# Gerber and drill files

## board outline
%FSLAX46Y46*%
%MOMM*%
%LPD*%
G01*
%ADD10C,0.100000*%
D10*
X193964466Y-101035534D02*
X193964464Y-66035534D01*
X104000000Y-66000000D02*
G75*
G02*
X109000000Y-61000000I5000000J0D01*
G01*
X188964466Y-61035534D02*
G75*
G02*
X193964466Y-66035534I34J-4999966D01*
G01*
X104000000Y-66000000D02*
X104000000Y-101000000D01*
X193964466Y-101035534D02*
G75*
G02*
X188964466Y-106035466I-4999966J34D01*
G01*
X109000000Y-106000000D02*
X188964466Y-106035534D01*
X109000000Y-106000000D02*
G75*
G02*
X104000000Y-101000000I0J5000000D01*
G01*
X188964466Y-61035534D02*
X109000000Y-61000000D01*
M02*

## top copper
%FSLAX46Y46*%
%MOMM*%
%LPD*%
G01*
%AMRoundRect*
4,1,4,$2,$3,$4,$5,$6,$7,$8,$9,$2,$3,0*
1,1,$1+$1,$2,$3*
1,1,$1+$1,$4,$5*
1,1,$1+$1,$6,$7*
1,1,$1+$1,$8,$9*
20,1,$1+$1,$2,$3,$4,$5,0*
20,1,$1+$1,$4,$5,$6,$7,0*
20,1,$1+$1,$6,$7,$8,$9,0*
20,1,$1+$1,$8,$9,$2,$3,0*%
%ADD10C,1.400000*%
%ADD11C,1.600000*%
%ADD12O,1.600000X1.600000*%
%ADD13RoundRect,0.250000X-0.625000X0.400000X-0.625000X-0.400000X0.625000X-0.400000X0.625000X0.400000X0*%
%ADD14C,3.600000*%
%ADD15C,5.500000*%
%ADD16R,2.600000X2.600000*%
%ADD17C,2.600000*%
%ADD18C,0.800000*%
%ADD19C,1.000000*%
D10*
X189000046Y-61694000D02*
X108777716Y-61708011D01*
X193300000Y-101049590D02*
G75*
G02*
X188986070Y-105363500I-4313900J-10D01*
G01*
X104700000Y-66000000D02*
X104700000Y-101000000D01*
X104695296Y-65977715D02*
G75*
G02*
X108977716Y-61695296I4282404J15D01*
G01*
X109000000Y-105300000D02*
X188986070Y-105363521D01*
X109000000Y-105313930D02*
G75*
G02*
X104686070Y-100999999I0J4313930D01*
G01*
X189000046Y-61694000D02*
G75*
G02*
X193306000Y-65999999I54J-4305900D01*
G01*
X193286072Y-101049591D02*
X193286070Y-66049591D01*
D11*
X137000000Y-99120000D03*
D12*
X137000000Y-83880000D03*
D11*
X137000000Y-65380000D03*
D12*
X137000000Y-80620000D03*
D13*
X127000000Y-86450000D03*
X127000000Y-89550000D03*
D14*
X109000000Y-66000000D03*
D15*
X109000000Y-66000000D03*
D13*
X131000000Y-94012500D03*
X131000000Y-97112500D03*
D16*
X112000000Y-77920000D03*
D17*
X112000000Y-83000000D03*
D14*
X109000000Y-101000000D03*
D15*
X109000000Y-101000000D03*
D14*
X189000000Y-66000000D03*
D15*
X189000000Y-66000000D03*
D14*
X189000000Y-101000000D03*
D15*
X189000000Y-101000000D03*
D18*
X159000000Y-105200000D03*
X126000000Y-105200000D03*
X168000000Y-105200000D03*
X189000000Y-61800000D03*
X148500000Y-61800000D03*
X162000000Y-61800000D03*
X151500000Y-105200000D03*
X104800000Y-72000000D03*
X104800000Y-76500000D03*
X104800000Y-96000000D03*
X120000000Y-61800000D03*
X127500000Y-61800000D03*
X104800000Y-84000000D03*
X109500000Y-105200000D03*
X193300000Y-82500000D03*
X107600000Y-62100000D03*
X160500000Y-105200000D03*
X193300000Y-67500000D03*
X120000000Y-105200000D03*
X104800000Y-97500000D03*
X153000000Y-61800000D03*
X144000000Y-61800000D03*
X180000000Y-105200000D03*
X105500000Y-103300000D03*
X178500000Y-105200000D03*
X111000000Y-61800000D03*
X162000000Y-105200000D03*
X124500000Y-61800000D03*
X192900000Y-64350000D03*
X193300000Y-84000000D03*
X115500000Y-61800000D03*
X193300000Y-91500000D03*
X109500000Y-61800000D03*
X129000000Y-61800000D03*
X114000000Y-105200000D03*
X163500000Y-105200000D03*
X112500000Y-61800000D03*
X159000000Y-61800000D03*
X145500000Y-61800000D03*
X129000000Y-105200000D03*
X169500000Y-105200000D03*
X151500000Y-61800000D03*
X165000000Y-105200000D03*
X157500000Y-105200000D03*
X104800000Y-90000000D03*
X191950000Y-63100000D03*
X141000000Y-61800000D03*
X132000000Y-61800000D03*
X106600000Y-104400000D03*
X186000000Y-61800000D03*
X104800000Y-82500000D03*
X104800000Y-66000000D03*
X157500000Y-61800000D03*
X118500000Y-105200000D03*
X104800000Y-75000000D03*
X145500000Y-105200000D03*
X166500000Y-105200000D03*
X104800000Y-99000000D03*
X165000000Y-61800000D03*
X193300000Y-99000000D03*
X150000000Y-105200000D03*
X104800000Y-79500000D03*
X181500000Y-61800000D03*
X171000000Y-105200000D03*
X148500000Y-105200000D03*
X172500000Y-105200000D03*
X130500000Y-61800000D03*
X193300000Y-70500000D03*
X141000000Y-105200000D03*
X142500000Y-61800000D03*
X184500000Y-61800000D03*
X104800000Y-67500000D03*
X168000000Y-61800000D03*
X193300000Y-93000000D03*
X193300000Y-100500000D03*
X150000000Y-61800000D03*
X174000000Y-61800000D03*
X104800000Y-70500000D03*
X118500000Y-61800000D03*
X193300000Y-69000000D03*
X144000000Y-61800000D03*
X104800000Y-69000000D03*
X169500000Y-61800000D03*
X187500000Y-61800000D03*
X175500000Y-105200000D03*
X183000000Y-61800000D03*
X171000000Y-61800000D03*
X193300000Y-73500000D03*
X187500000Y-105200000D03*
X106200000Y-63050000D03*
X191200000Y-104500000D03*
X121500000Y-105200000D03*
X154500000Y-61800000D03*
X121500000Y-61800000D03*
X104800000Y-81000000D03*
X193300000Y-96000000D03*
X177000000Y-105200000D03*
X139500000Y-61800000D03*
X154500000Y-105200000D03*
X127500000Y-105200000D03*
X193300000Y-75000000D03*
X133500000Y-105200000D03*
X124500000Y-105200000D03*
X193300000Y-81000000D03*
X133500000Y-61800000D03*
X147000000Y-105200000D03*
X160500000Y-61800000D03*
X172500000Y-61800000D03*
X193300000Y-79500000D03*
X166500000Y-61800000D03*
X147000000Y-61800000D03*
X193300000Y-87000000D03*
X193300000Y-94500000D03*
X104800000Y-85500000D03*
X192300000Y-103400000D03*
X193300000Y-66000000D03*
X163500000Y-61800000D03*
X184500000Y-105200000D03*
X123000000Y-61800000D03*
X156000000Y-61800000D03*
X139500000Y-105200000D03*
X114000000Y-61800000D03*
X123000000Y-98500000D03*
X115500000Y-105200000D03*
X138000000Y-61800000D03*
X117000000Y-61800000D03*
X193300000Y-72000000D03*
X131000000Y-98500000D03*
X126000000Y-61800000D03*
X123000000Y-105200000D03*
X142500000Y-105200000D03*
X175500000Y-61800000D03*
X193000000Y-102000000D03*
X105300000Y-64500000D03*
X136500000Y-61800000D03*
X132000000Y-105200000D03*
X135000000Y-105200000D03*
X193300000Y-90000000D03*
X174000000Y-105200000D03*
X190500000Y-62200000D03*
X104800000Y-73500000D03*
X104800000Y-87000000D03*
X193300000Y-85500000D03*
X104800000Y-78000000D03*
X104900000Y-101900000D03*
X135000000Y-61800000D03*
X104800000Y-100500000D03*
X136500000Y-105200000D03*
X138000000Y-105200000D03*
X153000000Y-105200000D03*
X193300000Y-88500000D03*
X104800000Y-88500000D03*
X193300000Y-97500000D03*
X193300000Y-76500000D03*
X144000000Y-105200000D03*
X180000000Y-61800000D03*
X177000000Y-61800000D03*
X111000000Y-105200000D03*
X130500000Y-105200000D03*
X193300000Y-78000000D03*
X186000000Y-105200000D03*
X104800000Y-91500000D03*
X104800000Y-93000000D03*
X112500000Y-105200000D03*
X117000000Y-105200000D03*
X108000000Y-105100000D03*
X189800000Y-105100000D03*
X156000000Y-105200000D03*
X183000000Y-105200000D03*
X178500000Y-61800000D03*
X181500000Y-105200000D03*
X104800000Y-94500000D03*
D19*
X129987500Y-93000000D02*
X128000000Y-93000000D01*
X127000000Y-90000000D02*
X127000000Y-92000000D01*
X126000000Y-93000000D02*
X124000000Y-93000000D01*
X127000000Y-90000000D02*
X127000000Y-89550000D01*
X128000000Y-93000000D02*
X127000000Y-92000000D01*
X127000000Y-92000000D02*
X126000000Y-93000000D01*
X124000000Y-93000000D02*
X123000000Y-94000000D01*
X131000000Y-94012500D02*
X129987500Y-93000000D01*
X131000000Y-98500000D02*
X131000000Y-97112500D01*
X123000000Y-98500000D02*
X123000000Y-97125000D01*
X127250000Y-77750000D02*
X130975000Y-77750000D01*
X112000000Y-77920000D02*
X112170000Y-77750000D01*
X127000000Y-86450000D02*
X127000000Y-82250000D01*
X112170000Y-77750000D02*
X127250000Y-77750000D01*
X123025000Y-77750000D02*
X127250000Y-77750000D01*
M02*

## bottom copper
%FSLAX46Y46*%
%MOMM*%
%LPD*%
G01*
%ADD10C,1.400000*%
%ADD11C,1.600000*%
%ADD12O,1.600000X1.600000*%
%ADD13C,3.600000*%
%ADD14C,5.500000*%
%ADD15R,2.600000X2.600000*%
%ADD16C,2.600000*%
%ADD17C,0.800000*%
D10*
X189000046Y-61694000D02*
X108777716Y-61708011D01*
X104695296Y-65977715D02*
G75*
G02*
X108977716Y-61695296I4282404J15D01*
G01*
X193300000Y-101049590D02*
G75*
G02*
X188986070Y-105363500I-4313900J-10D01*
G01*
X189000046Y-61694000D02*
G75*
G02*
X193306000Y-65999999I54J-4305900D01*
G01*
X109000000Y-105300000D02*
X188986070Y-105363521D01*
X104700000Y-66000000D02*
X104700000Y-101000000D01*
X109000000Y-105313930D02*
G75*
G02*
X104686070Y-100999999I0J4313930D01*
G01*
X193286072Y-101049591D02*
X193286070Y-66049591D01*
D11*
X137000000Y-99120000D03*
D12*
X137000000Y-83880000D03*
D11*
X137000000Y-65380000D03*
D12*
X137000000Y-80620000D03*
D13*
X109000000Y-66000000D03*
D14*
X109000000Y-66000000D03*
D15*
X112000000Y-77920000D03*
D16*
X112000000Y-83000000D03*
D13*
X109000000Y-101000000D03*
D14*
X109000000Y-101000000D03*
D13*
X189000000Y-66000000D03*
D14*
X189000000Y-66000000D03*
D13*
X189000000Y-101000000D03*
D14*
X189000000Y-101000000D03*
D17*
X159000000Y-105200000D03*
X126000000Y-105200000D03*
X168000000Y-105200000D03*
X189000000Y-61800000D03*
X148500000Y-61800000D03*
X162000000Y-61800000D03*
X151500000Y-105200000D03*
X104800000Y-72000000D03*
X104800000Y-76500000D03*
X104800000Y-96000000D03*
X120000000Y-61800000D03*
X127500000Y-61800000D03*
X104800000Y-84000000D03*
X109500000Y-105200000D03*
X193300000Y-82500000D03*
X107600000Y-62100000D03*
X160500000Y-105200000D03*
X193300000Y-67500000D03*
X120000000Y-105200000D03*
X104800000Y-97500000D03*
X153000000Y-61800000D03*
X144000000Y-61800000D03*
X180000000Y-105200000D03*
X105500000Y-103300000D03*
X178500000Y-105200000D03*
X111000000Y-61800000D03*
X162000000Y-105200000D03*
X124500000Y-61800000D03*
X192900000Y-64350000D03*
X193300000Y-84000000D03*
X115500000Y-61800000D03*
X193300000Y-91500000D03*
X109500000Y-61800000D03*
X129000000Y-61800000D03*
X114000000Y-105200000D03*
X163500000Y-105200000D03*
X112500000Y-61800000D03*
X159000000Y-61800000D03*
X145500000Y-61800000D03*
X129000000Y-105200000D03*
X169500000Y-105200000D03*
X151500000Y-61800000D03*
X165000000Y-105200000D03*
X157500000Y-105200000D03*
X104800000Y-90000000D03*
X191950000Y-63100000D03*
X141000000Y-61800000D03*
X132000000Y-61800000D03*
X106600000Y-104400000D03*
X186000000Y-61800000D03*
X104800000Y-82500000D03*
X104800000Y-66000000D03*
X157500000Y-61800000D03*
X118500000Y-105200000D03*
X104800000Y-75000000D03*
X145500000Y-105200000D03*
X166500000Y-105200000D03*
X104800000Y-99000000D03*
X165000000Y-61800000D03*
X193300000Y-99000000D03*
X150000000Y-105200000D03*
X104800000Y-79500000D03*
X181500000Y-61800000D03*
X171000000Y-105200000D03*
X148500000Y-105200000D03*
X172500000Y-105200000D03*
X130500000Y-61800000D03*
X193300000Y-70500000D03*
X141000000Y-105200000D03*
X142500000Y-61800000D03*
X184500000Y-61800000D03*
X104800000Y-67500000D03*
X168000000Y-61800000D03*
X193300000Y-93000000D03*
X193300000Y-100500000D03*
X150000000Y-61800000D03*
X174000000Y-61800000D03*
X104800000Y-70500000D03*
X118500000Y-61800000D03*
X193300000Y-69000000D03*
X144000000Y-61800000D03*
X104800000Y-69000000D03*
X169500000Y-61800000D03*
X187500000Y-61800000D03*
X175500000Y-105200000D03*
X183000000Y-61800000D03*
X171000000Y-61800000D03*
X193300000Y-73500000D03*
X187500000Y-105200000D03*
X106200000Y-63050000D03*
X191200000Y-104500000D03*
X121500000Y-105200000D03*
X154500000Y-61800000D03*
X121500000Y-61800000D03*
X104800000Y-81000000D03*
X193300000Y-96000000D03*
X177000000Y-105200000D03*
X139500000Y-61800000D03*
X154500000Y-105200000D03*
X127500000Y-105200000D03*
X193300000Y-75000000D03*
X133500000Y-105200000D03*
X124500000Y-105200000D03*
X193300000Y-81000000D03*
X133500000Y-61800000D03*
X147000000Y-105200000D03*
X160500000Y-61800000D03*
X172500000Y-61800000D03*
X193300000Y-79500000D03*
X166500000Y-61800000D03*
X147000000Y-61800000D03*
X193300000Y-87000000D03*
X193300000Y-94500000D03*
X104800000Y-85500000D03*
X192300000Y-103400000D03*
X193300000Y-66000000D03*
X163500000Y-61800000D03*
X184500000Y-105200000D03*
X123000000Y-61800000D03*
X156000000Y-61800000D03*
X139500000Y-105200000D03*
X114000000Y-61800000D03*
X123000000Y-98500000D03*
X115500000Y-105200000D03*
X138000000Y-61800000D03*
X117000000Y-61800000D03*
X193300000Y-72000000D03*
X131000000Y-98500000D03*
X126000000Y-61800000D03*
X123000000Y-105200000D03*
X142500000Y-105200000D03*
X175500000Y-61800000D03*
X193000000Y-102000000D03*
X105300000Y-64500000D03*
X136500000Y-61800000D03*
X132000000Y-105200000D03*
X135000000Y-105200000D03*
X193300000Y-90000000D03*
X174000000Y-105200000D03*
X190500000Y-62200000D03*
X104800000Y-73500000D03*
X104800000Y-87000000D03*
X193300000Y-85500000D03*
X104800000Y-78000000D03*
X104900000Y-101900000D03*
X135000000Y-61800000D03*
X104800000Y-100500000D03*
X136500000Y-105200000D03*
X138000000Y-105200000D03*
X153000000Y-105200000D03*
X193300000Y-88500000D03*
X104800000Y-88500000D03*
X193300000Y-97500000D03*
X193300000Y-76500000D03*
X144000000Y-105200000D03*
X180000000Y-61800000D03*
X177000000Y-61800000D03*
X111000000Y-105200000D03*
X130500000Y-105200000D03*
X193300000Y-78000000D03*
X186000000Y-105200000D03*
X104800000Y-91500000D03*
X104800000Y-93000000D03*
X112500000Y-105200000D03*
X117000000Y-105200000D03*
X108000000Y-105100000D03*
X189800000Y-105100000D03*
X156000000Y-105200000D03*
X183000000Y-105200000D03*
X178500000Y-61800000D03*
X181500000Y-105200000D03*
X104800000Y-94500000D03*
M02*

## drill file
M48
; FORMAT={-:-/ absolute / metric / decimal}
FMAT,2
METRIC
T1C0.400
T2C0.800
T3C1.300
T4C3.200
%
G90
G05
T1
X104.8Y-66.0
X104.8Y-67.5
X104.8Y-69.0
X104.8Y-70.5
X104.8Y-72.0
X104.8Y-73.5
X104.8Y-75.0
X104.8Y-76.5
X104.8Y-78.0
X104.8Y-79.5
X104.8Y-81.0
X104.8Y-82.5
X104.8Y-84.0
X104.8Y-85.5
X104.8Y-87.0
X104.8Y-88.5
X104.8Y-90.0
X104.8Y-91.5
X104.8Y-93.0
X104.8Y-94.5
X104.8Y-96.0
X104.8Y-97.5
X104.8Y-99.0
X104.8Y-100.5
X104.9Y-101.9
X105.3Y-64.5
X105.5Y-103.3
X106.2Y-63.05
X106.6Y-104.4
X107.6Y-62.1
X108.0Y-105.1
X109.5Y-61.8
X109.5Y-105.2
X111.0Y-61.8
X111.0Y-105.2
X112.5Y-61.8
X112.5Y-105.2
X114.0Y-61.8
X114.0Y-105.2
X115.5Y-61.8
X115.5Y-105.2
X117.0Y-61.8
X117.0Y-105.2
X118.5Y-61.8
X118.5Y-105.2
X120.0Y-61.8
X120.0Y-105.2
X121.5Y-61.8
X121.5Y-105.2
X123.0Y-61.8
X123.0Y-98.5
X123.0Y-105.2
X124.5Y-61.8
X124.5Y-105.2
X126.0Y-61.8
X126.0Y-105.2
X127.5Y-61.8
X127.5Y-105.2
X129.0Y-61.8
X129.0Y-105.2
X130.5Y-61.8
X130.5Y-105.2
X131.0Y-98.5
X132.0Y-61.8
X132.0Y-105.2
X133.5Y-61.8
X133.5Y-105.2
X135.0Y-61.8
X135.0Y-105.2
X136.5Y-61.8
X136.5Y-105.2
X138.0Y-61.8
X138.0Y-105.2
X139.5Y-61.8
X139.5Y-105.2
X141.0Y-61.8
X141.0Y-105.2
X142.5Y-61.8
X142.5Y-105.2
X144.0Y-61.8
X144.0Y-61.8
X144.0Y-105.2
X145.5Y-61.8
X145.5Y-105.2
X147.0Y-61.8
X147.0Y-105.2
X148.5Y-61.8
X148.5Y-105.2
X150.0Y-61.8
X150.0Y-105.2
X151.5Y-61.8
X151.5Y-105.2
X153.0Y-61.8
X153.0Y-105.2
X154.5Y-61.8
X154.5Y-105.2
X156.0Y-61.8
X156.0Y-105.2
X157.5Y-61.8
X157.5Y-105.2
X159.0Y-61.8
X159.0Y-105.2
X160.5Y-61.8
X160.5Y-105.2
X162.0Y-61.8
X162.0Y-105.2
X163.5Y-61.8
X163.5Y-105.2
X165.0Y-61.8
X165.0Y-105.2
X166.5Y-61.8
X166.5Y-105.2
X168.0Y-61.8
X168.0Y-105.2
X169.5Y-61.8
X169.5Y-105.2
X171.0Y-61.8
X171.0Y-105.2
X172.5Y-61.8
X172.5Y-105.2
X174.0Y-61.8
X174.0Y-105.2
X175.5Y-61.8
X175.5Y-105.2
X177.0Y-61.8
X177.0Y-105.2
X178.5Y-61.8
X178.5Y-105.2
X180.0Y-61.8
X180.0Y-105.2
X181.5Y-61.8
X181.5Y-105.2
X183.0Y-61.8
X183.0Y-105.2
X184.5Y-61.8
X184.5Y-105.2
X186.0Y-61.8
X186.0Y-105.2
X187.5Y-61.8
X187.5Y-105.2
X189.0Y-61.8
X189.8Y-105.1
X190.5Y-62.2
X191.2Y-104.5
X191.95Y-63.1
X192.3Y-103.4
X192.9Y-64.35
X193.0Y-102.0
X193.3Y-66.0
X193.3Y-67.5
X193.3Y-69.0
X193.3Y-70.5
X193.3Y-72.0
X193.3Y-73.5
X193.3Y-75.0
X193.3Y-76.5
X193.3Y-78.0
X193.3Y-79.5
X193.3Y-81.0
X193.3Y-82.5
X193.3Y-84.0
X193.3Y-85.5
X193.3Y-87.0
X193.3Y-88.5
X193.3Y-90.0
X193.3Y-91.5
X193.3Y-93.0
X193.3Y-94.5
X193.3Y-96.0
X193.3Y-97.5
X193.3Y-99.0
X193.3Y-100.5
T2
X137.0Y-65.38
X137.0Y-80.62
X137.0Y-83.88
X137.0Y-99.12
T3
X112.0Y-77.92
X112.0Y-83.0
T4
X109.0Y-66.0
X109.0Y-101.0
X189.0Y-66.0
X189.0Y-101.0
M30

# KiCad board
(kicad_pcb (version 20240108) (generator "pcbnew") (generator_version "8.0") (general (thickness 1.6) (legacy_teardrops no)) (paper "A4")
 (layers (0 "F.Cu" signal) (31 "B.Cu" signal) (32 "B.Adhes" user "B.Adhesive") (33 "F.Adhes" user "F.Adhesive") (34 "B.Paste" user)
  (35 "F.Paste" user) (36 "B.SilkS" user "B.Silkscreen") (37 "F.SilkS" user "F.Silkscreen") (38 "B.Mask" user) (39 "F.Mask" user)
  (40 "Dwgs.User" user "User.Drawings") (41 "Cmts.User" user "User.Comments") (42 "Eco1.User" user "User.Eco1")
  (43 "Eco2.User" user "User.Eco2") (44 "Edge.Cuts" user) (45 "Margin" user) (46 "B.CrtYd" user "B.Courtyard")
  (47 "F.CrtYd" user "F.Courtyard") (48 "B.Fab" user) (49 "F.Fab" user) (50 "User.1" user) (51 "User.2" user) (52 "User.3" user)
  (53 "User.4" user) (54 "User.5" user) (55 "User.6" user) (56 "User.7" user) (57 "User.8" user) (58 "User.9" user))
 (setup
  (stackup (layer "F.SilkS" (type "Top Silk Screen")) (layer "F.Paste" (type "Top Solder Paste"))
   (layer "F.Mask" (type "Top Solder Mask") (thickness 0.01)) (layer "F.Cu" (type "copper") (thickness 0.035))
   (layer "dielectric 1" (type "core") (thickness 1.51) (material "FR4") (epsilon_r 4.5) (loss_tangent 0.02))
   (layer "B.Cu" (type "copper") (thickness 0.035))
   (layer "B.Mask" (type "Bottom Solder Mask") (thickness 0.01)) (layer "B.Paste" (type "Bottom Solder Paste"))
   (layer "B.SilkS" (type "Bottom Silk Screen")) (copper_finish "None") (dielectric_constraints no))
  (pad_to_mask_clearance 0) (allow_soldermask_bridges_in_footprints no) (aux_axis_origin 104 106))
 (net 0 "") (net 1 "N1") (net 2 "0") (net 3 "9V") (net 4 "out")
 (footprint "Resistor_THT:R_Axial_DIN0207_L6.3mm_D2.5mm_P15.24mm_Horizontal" (layer "F.Cu") (at 137 99.12 90)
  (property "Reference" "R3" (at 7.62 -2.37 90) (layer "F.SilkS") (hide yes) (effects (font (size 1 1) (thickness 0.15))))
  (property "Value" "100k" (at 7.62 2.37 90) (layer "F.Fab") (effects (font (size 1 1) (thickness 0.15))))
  (pad "1" thru_hole circle (at 0 0 90) (size 1.6 1.6) (drill 0.8) (layers "*.Cu" "*.Mask") (remove_unused_layers no) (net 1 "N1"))
  (pad "2" thru_hole oval (at 15.24 0 90) (size 1.6 1.6) (drill 0.8) (layers "*.Cu" "*.Mask") (remove_unused_layers no) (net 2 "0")))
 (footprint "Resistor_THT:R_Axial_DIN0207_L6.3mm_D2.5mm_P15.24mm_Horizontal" (layer "F.Cu") (at 137 65.38 -90)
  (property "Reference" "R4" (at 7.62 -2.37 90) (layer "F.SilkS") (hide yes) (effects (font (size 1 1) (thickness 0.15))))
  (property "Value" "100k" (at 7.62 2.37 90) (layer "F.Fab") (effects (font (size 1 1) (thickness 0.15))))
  (pad "1" thru_hole circle (at 0 0 270) (size 1.6 1.6) (drill 0.8) (layers "*.Cu" "*.Mask") (remove_unused_layers no) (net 1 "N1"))
  (pad "2" thru_hole oval (at 15.24 0 270) (size 1.6 1.6) (drill 0.8) (layers "*.Cu" "*.Mask") (remove_unused_layers no) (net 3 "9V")))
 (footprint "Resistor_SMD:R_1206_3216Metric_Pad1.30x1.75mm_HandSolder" (layer "F.Cu") (at 127 88 -90)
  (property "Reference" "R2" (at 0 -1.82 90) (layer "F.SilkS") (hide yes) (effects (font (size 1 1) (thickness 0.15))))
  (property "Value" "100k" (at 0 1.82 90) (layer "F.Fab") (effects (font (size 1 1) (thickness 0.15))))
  (pad "1" smd roundrect (at -1.55 0 270) (size 1.3 1.75) (layers "F.Cu" "F.Paste" "F.Mask") (roundrect_rratio 0.1923076923) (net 3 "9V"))
  (pad "2" smd roundrect (at 1.55 0 270) (size 1.3 1.75) (layers "F.Cu" "F.Paste" "F.Mask") (roundrect_rratio 0.1923076923) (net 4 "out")))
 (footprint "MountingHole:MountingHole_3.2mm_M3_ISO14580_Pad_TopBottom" (layer "F.Cu") (at 109 66)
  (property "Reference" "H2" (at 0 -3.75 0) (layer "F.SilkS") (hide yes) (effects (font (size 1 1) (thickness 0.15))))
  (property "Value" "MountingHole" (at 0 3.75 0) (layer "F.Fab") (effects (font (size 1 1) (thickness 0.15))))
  (pad "1" thru_hole circle (at 0 0) (size 3.6 3.6) (drill 3.2) (layers "*.Cu" "*.Mask") (remove_unused_layers no))
  (pad "1" connect circle (at 0 0) (size 5.5 5.5) (layers "F.Cu" "F.Mask"))
  (pad "1" connect circle (at 0 0) (size 5.5 5.5) (layers "B.Cu" "B.Mask")))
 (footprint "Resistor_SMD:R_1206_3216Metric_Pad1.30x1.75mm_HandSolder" (layer "F.Cu") (at 131 95.5625 -90)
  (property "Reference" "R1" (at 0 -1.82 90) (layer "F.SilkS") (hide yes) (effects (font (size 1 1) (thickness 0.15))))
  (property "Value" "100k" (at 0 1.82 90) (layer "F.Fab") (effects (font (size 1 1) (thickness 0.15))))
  (pad "1" smd roundrect (at -1.55 0 270) (size 1.3 1.75) (layers "F.Cu" "F.Paste" "F.Mask") (roundrect_rratio 0.1923076923) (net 4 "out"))
  (pad "2" smd roundrect (at 1.55 0 270) (size 1.3 1.75) (layers "F.Cu" "F.Paste" "F.Mask") (roundrect_rratio 0.1923076923) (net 2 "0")))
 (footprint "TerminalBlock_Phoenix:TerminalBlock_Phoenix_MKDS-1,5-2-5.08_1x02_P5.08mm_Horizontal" (layer "F.Cu") (at 112 77.92 -90)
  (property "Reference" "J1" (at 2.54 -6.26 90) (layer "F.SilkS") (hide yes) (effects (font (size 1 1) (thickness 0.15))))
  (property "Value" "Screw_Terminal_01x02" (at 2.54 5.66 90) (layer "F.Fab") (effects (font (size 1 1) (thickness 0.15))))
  (pad "1" thru_hole rect (at 0 0 270) (size 2.6 2.6) (drill 1.3) (layers "*.Cu" "*.Mask") (remove_unused_layers no) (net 3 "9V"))
  (pad "2" thru_hole circle (at 5.08 0 270) (size 2.6 2.6) (drill 1.3) (layers "*.Cu" "*.Mask") (remove_unused_layers no) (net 2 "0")))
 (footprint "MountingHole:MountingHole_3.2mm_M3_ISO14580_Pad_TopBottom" (layer "F.Cu") (at 109 101 -90)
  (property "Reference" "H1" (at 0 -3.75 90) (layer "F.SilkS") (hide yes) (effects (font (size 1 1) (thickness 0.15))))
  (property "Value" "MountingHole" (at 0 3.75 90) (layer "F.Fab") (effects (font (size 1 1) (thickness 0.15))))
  (pad "1" thru_hole circle (at 0 0 270) (size 3.6 3.6) (drill 3.2) (layers "*.Cu" "*.Mask") (remove_unused_layers no))
  (pad "1" connect circle (at 0 0 270) (size 5.5 5.5) (layers "F.Cu" "F.Mask"))
  (pad "1" connect circle (at 0 0 270) (size 5.5 5.5) (layers "B.Cu" "B.Mask")))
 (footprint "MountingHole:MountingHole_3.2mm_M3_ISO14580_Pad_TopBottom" (layer "F.Cu") (at 189 66)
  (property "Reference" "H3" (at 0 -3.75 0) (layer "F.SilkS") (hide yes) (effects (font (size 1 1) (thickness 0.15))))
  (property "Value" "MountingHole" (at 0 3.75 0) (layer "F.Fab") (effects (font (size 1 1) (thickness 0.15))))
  (pad "1" thru_hole circle (at 0 0) (size 3.6 3.6) (drill 3.2) (layers "*.Cu" "*.Mask") (remove_unused_layers no))
  (pad "1" connect circle (at 0 0) (size 5.5 5.5) (layers "F.Cu" "F.Mask"))
  (pad "1" connect circle (at 0 0) (size 5.5 5.5) (layers "B.Cu" "B.Mask")))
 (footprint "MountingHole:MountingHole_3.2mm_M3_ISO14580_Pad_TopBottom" (layer "F.Cu") (at 189 101)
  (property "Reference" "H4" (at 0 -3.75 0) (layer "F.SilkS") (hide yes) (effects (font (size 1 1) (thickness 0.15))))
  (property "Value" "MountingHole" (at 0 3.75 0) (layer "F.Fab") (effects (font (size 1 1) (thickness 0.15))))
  (pad "1" thru_hole circle (at 0 0) (size 3.6 3.6) (drill 3.2) (layers "*.Cu" "*.Mask") (remove_unused_layers no))
  (pad "1" connect circle (at 0 0) (size 5.5 5.5) (layers "F.Cu" "F.Mask"))
  (pad "1" connect circle (at 0 0) (size 5.5 5.5) (layers "B.Cu" "B.Mask")))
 (gr_line (start 189.000046 61.694) (end 108.777716 61.708011) (stroke (width 1.4) (type default)) (layer "F.Cu") (net 2))
 (gr_arc (start 193.3 101.04959) (mid 192.036477 104.099991) (end 188.98607 105.363521) (stroke (width 1.4) (type default)) (layer "F.Cu")
  (net 2))
 (gr_line (start 104.7 66) (end 104.7 101) (stroke (width 1.4) (type default)) (layer "F.Cu") (net 2))
 (gr_arc (start 104.695296 65.977715) (mid 105.949583 62.949583) (end 108.977716 61.695296) (stroke (width 1.4) (type default))
  (layer "F.Cu") (net 2))
 (gr_line (start 109 105.3) (end 188.98607 105.363521) (stroke (width 1.4) (type default)) (layer "F.Cu") (net 2))
 (gr_arc (start 109 105.31393) (mid 105.949588 104.05041) (end 104.68607 100.999999) (stroke (width 1.4) (type default)) (layer "F.Cu")
  (net 2))
 (gr_arc (start 189.000046 61.694) (mid 192.04487 62.955184) (end 193.306046 65.999999) (stroke (width 1.4) (type default)) (layer "F.Cu")
  (net 2))
 (gr_line (start 193.286072 101.049591) (end 193.28607 66.049591) (stroke (width 1.4) (type default)) (layer "F.Cu") (net 2))
 (gr_line (start 189.000046 61.694) (end 108.777716 61.708011) (stroke (width 1.4) (type default)) (layer "B.Cu") (net 2))
 (gr_arc (start 104.695296 65.977715) (mid 105.949583 62.949583) (end 108.977716 61.695296) (stroke (width 1.4) (type default))
  (layer "B.Cu") (net 2))
 (gr_arc (start 193.3 101.04959) (mid 192.036477 104.099991) (end 188.98607 105.363521) (stroke (width 1.4) (type default)) (layer "B.Cu")
  (net 2))
 (gr_arc (start 189.000046 61.694) (mid 192.04487 62.955184) (end 193.306046 65.999999) (stroke (width 1.4) (type default)) (layer "B.Cu")
  (net 2))
 (gr_line (start 109 105.3) (end 188.98607 105.363521) (stroke (width 1.4) (type default)) (layer "B.Cu") (net 2))
 (gr_line (start 104.7 66) (end 104.7 101) (stroke (width 1.4) (type default)) (layer "B.Cu") (net 2))
 (gr_arc (start 109 105.31393) (mid 105.949588 104.05041) (end 104.68607 100.999999) (stroke (width 1.4) (type default)) (layer "B.Cu")
  (net 2))
 (gr_line (start 193.286072 101.049591) (end 193.28607 66.049591) (stroke (width 1.4) (type default)) (layer "B.Cu") (net 2))
 (gr_line (start 193.964466 101.035534) (end 193.964464 66.035534) (stroke (width 0.1) (type default)) (layer "Edge.Cuts"))
 (gr_arc (start 104 66) (mid 105.464467 62.464467) (end 109 61) (stroke (width 0.1) (type default)) (layer "Edge.Cuts"))
 (gr_arc (start 188.964466 61.035534) (mid 192.5 62.5) (end 193.964464 66.035534) (stroke (width 0.1) (type default)) (layer "Edge.Cuts"))
 (gr_line (start 104 66) (end 104 101) (stroke (width 0.1) (type default)) (layer "Edge.Cuts"))
 (gr_arc (start 193.964466 101.035534) (mid 192.5 104.571068) (end 188.964466 106.035534) (stroke (width 0.1) (type default))
  (layer "Edge.Cuts"))
 (gr_line (start 109 106) (end 188.964466 106.035534) (stroke (width 0.1) (type default)) (layer "Edge.Cuts"))
 (gr_arc (start 109 106) (mid 105.464467 104.535533) (end 104 101) (stroke (width 0.1) (type default)) (layer "Edge.Cuts"))
 (gr_line (start 188.964466 61.035534) (end 109 61) (stroke (width 0.1) (type default)) (layer "Edge.Cuts"))
 (segment (start 129.9875 93) (end 128 93) (width 1) (layer "F.Cu") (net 4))
 (segment (start 127 90) (end 127 92) (width 1) (layer "F.Cu") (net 4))
 (segment (start 126 93) (end 124 93) (width 1) (layer "F.Cu") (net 4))
 (segment (start 127 90) (end 127 89.55) (width 1) (layer "F.Cu") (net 4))
 (segment (start 128 93) (end 127 92) (width 1) (layer "F.Cu") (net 4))
 (segment (start 127 92) (end 126 93) (width 1) (layer "F.Cu") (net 4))
 (segment (start 124 93) (end 123 94) (width 1) (layer "F.Cu") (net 4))
 (segment (start 131 94.0125) (end 129.9875 93) (width 1) (layer "F.Cu") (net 4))
 (segment (start 131 98.5) (end 131 97.1125) (width 1) (layer "F.Cu") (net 2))
 (segment (start 123 98.5) (end 123 97.125) (width 1) (layer "F.Cu") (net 2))
 (via (at 159 105.2) (size 0.8) (drill 0.4) (layers "F.Cu" "B.Cu") (free yes) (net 2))
 (via (at 126 105.2) (size 0.8) (drill 0.4) (layers "F.Cu" "B.Cu") (free yes) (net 2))
 (via (at 168 105.2) (size 0.8) (drill 0.4) (layers "F.Cu" "B.Cu") (free yes) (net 2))
 (via (at 189 61.8) (size 0.8) (drill 0.4) (layers "F.Cu" "B.Cu") (free yes) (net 2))
 (via (at 148.5 61.8) (size 0.8) (drill 0.4) (layers "F.Cu" "B.Cu") (free yes) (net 2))
 (via (at 162 61.8) (size 0.8) (drill 0.4) (layers "F.Cu" "B.Cu") (free yes) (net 2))
 (via (at 151.5 105.2) (size 0.8) (drill 0.4) (layers "F.Cu" "B.Cu") (free yes) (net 2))
 (via (at 104.8 72) (size 0.8) (drill 0.4) (layers "F.Cu" "B.Cu") (free yes) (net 2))
 (via (at 104.8 76.5) (size 0.8) (drill 0.4) (layers "F.Cu" "B.Cu") (free yes) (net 2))
 (via (at 104.8 96) (size 0.8) (drill 0.4) (layers "F.Cu" "B.Cu") (free yes) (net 2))
 (via (at 120 61.8) (size 0.8) (drill 0.4) (layers "F.Cu" "B.Cu") (free yes) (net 2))
 (via (at 127.5 61.8) (size 0.8) (drill 0.4) (layers "F.Cu" "B.Cu") (free yes) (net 2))
 (via (at 104.8 84) (size 0.8) (drill 0.4) (layers "F.Cu" "B.Cu") (free yes) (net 2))
 (via (at 109.5 105.2) (size 0.8) (drill 0.4) (layers "F.Cu" "B.Cu") (free yes) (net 2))
 (via (at 193.3 82.5) (size 0.8) (drill 0.4) (layers "F.Cu" "B.Cu") (free yes) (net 2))
 (via (at 107.6 62.1) (size 0.8) (drill 0.4) (layers "F.Cu" "B.Cu") (free yes) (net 2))
 (via (at 160.5 105.2) (size 0.8) (drill 0.4) (layers "F.Cu" "B.Cu") (free yes) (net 2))
 (via (at 193.3 67.5) (size 0.8) (drill 0.4) (layers "F.Cu" "B.Cu") (free yes) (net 2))
 (via (at 120 105.2) (size 0.8) (drill 0.4) (layers "F.Cu" "B.Cu") (free yes) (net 2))
 (via (at 104.8 97.5) (size 0.8) (drill 0.4) (layers "F.Cu" "B.Cu") (free yes) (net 2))
 (via (at 153 61.8) (size 0.8) (drill 0.4) (layers "F.Cu" "B.Cu") (free yes) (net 2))
 (via (at 144 61.8) (size 0.8) (drill 0.4) (layers "F.Cu" "B.Cu") (free yes) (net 2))
 (via (at 180 105.2) (size 0.8) (drill 0.4) (layers "F.Cu" "B.Cu") (free yes) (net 2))
 (via (at 105.5 103.3) (size 0.8) (drill 0.4) (layers "F.Cu" "B.Cu") (free yes) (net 2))
 (via (at 178.5 105.2) (size 0.8) (drill 0.4) (layers "F.Cu" "B.Cu") (free yes) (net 2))
 (via (at 111 61.8) (size 0.8) (drill 0.4) (layers "F.Cu" "B.Cu") (free yes) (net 2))
 (via (at 162 105.2) (size 0.8) (drill 0.4) (layers "F.Cu" "B.Cu") (free yes) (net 2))
 (via (at 124.5 61.8) (size 0.8) (drill 0.4) (layers "F.Cu" "B.Cu") (free yes) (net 2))
 (via (at 192.9 64.35) (size 0.8) (drill 0.4) (layers "F.Cu" "B.Cu") (free yes) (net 2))
 (via (at 193.3 84) (size 0.8) (drill 0.4) (layers "F.Cu" "B.Cu") (free yes) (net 2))
 (via (at 115.5 61.8) (size 0.8) (drill 0.4) (layers "F.Cu" "B.Cu") (free yes) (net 2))
 (via (at 193.3 91.5) (size 0.8) (drill 0.4) (layers "F.Cu" "B.Cu") (free yes) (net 2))
 (via (at 109.5 61.8) (size 0.8) (drill 0.4) (layers "F.Cu" "B.Cu") (free yes) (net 2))
 (via (at 129 61.8) (size 0.8) (drill 0.4) (layers "F.Cu" "B.Cu") (free yes) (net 2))
 (via (at 114 105.2) (size 0.8) (drill 0.4) (layers "F.Cu" "B.Cu") (free yes) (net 2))
 (via (at 163.5 105.2) (size 0.8) (drill 0.4) (layers "F.Cu" "B.Cu") (free yes) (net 2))
 (via (at 112.5 61.8) (size 0.8) (drill 0.4) (layers "F.Cu" "B.Cu") (free yes) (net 2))
 (via (at 159 61.8) (size 0.8) (drill 0.4) (layers "F.Cu" "B.Cu") (free yes) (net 2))
 (via (at 145.5 61.8) (size 0.8) (drill 0.4) (layers "F.Cu" "B.Cu") (free yes) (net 2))
 (via (at 129 105.2) (size 0.8) (drill 0.4) (layers "F.Cu" "B.Cu") (free yes) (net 2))
 (via (at 169.5 105.2) (size 0.8) (drill 0.4) (layers "F.Cu" "B.Cu") (free yes) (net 2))
 (via (at 151.5 61.8) (size 0.8) (drill 0.4) (layers "F.Cu" "B.Cu") (free yes) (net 2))
 (via (at 165 105.2) (size 0.8) (drill 0.4) (layers "F.Cu" "B.Cu") (free yes) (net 2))
 (via (at 157.5 105.2) (size 0.8) (drill 0.4) (layers "F.Cu" "B.Cu") (free yes) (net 2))
 (via (at 104.8 90) (size 0.8) (drill 0.4) (layers "F.Cu" "B.Cu") (free yes) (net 2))
 (via (at 191.95 63.1) (size 0.8) (drill 0.4) (layers "F.Cu" "B.Cu") (free yes) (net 2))
 (via (at 141 61.8) (size 0.8) (drill 0.4) (layers "F.Cu" "B.Cu") (free yes) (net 2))
 (via (at 132 61.8) (size 0.8) (drill 0.4) (layers "F.Cu" "B.Cu") (free yes) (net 2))
 (via (at 106.6 104.4) (size 0.8) (drill 0.4) (layers "F.Cu" "B.Cu") (free yes) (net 2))
 (via (at 186 61.8) (size 0.8) (drill 0.4) (layers "F.Cu" "B.Cu") (free yes) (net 2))
 (via (at 104.8 82.5) (size 0.8) (drill 0.4) (layers "F.Cu" "B.Cu") (free yes) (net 2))
 (via (at 104.8 66) (size 0.8) (drill 0.4) (layers "F.Cu" "B.Cu") (free yes) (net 2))
 (via (at 157.5 61.8) (size 0.8) (drill 0.4) (layers "F.Cu" "B.Cu") (free yes) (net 2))
 (via (at 118.5 105.2) (size 0.8) (drill 0.4) (layers "F.Cu" "B.Cu") (free yes) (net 2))
 (via (at 104.8 75) (size 0.8) (drill 0.4) (layers "F.Cu" "B.Cu") (free yes) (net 2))
 (via (at 145.5 105.2) (size 0.8) (drill 0.4) (layers "F.Cu" "B.Cu") (free yes) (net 2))
 (via (at 166.5 105.2) (size 0.8) (drill 0.4) (layers "F.Cu" "B.Cu") (free yes) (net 2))
 (via (at 104.8 99) (size 0.8) (drill 0.4) (layers "F.Cu" "B.Cu") (free yes) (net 2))
 (via (at 165 61.8) (size 0.8) (drill 0.4) (layers "F.Cu" "B.Cu") (free yes) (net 2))
 (via (at 193.3 99) (size 0.8) (drill 0.4) (layers "F.Cu" "B.Cu") (free yes) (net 2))
 (via (at 150 105.2) (size 0.8) (drill 0.4) (layers "F.Cu" "B.Cu") (free yes) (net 2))
 (via (at 104.8 79.5) (size 0.8) (drill 0.4) (layers "F.Cu" "B.Cu") (free yes) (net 2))
 (via (at 181.5 61.8) (size 0.8) (drill 0.4) (layers "F.Cu" "B.Cu") (free yes) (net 2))
 (via (at 171 105.2) (size 0.8) (drill 0.4) (layers "F.Cu" "B.Cu") (free yes) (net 2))
 (via (at 148.5 105.2) (size 0.8) (drill 0.4) (layers "F.Cu" "B.Cu") (free yes) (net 2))
 (via (at 172.5 105.2) (size 0.8) (drill 0.4) (layers "F.Cu" "B.Cu") (free yes) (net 2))
 (via (at 130.5 61.8) (size 0.8) (drill 0.4) (layers "F.Cu" "B.Cu") (free yes) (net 2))
 (via (at 193.3 70.5) (size 0.8) (drill 0.4) (layers "F.Cu" "B.Cu") (free yes) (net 2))
 (via (at 141 105.2) (size 0.8) (drill 0.4) (layers "F.Cu" "B.Cu") (free yes) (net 2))
 (via (at 142.5 61.8) (size 0.8) (drill 0.4) (layers "F.Cu" "B.Cu") (free yes) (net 2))
 (via (at 184.5 61.8) (size 0.8) (drill 0.4) (layers "F.Cu" "B.Cu") (free yes) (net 2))
 (via (at 104.8 67.5) (size 0.8) (drill 0.4) (layers "F.Cu" "B.Cu") (free yes) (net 2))
 (via (at 168 61.8) (size 0.8) (drill 0.4) (layers "F.Cu" "B.Cu") (free yes) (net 2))
 (via (at 193.3 93) (size 0.8) (drill 0.4) (layers "F.Cu" "B.Cu") (free yes) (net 2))
 (via (at 193.3 100.5) (size 0.8) (drill 0.4) (layers "F.Cu" "B.Cu") (free yes) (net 2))
 (via (at 150 61.8) (size 0.8) (drill 0.4) (layers "F.Cu" "B.Cu") (free yes) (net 2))
 (via (at 174 61.8) (size 0.8) (drill 0.4) (layers "F.Cu" "B.Cu") (free yes) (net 2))
 (via (at 104.8 70.5) (size 0.8) (drill 0.4) (layers "F.Cu" "B.Cu") (free yes) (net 2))
 (via (at 118.5 61.8) (size 0.8) (drill 0.4) (layers "F.Cu" "B.Cu") (free yes) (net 2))
 (via (at 193.3 69) (size 0.8) (drill 0.4) (layers "F.Cu" "B.Cu") (free yes) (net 2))
 (via (at 144 61.8) (size 0.8) (drill 0.4) (layers "F.Cu" "B.Cu") (free yes) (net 2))
 (via (at 104.8 69) (size 0.8) (drill 0.4) (layers "F.Cu" "B.Cu") (free yes) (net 2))
 (via (at 169.5 61.8) (size 0.8) (drill 0.4) (layers "F.Cu" "B.Cu") (free yes) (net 2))
 (via (at 187.5 61.8) (size 0.8) (drill 0.4) (layers "F.Cu" "B.Cu") (free yes) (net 2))
 (via (at 175.5 105.2) (size 0.8) (drill 0.4) (layers "F.Cu" "B.Cu") (free yes) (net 2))
 (via (at 183 61.8) (size 0.8) (drill 0.4) (layers "F.Cu" "B.Cu") (free yes) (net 2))
 (via (at 171 61.8) (size 0.8) (drill 0.4) (layers "F.Cu" "B.Cu") (free yes) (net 2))
 (via (at 193.3 73.5) (size 0.8) (drill 0.4) (layers "F.Cu" "B.Cu") (free yes) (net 2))
 (via (at 187.5 105.2) (size 0.8) (drill 0.4) (layers "F.Cu" "B.Cu") (free yes) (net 2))
 (via (at 106.2 63.05) (size 0.8) (drill 0.4) (layers "F.Cu" "B.Cu") (free yes) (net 2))
 (via (at 191.2 104.5) (size 0.8) (drill 0.4) (layers "F.Cu" "B.Cu") (free yes) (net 2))
 (via (at 121.5 105.2) (size 0.8) (drill 0.4) (layers "F.Cu" "B.Cu") (free yes) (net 2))
 (via (at 154.5 61.8) (size 0.8) (drill 0.4) (layers "F.Cu" "B.Cu") (free yes) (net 2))
 (via (at 121.5 61.8) (size 0.8) (drill 0.4) (layers "F.Cu" "B.Cu") (free yes) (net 2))
 (via (at 104.8 81) (size 0.8) (drill 0.4) (layers "F.Cu" "B.Cu") (free yes) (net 2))
 (via (at 193.3 96) (size 0.8) (drill 0.4) (layers "F.Cu" "B.Cu") (free yes) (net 2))
 (via (at 177 105.2) (size 0.8) (drill 0.4) (layers "F.Cu" "B.Cu") (free yes) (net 2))
 (via (at 139.5 61.8) (size 0.8) (drill 0.4) (layers "F.Cu" "B.Cu") (free yes) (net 2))
 (via (at 154.5 105.2) (size 0.8) (drill 0.4) (layers "F.Cu" "B.Cu") (free yes) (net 2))
 (via (at 127.5 105.2) (size 0.8) (drill 0.4) (layers "F.Cu" "B.Cu") (free yes) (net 2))
 (via (at 193.3 75) (size 0.8) (drill 0.4) (layers "F.Cu" "B.Cu") (free yes) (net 2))
 (via (at 133.5 105.2) (size 0.8) (drill 0.4) (layers "F.Cu" "B.Cu") (free yes) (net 2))
 (via (at 124.5 105.2) (size 0.8) (drill 0.4) (layers "F.Cu" "B.Cu") (free yes) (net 2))
 (via (at 193.3 81) (size 0.8) (drill 0.4) (layers "F.Cu" "B.Cu") (free yes) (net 2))
 (via (at 133.5 61.8) (size 0.8) (drill 0.4) (layers "F.Cu" "B.Cu") (free yes) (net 2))
 (via (at 147 105.2) (size 0.8) (drill 0.4) (layers "F.Cu" "B.Cu") (free yes) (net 2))
 (via (at 160.5 61.8) (size 0.8) (drill 0.4) (layers "F.Cu" "B.Cu") (free yes) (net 2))
 (via (at 172.5 61.8) (size 0.8) (drill 0.4) (layers "F.Cu" "B.Cu") (free yes) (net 2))
 (via (at 193.3 79.5) (size 0.8) (drill 0.4) (layers "F.Cu" "B.Cu") (free yes) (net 2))
 (via (at 166.5 61.8) (size 0.8) (drill 0.4) (layers "F.Cu" "B.Cu") (free yes) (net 2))
 (via (at 147 61.8) (size 0.8) (drill 0.4) (layers "F.Cu" "B.Cu") (free yes) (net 2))
 (via (at 193.3 87) (size 0.8) (drill 0.4) (layers "F.Cu" "B.Cu") (free yes) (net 2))
 (via (at 193.3 94.5) (size 0.8) (drill 0.4) (layers "F.Cu" "B.Cu") (free yes) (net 2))
 (via (at 104.8 85.5) (size 0.8) (drill 0.4) (layers "F.Cu" "B.Cu") (free yes) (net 2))
 (via (at 192.3 103.4) (size 0.8) (drill 0.4) (layers "F.Cu" "B.Cu") (free yes) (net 2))
 (via (at 193.3 66) (size 0.8) (drill 0.4) (layers "F.Cu" "B.Cu") (free yes) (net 2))
 (via (at 163.5 61.8) (size 0.8) (drill 0.4) (layers "F.Cu" "B.Cu") (free yes) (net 2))
 (via (at 184.5 105.2) (size 0.8) (drill 0.4) (layers "F.Cu" "B.Cu") (free yes) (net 2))
 (via (at 123 61.8) (size 0.8) (drill 0.4) (layers "F.Cu" "B.Cu") (free yes) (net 2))
 (via (at 156 61.8) (size 0.8) (drill 0.4) (layers "F.Cu" "B.Cu") (free yes) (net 2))
 (via (at 139.5 105.2) (size 0.8) (drill 0.4) (layers "F.Cu" "B.Cu") (free yes) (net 2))
 (via (at 114 61.8) (size 0.8) (drill 0.4) (layers "F.Cu" "B.Cu") (free yes) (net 2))
 (via (at 123 98.5) (size 0.8) (drill 0.4) (layers "F.Cu" "B.Cu") (free yes) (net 2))
 (via (at 115.5 105.2) (size 0.8) (drill 0.4) (layers "F.Cu" "B.Cu") (free yes) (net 2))
 (via (at 138 61.8) (size 0.8) (drill 0.4) (layers "F.Cu" "B.Cu") (free yes) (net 2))
 (via (at 117 61.8) (size 0.8) (drill 0.4) (layers "F.Cu" "B.Cu") (free yes) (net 2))
 (via (at 193.3 72) (size 0.8) (drill 0.4) (layers "F.Cu" "B.Cu") (free yes) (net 2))
 (via (at 131 98.5) (size 0.8) (drill 0.4) (layers "F.Cu" "B.Cu") (free yes) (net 2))
 (via (at 126 61.8) (size 0.8) (drill 0.4) (layers "F.Cu" "B.Cu") (free yes) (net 2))
 (via (at 123 105.2) (size 0.8) (drill 0.4) (layers "F.Cu" "B.Cu") (free yes) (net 2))
 (via (at 142.5 105.2) (size 0.8) (drill 0.4) (layers "F.Cu" "B.Cu") (free yes) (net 2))
 (via (at 175.5 61.8) (size 0.8) (drill 0.4) (layers "F.Cu" "B.Cu") (free yes) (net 2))
 (via (at 193 102) (size 0.8) (drill 0.4) (layers "F.Cu" "B.Cu") (free yes) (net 2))
 (via (at 105.3 64.5) (size 0.8) (drill 0.4) (layers "F.Cu" "B.Cu") (free yes) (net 2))
 (via (at 136.5 61.8) (size 0.8) (drill 0.4) (layers "F.Cu" "B.Cu") (free yes) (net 2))
 (via (at 132 105.2) (size 0.8) (drill 0.4) (layers "F.Cu" "B.Cu") (free yes) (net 2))
 (via (at 135 105.2) (size 0.8) (drill 0.4) (layers "F.Cu" "B.Cu") (free yes) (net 2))
 (via (at 193.3 90) (size 0.8) (drill 0.4) (layers "F.Cu" "B.Cu") (free yes) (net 2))
 (via (at 174 105.2) (size 0.8) (drill 0.4) (layers "F.Cu" "B.Cu") (free yes) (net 2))
 (via (at 190.5 62.2) (size 0.8) (drill 0.4) (layers "F.Cu" "B.Cu") (free yes) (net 2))
 (via (at 104.8 73.5) (size 0.8) (drill 0.4) (layers "F.Cu" "B.Cu") (free yes) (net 2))
 (via (at 104.8 87) (size 0.8) (drill 0.4) (layers "F.Cu" "B.Cu") (free yes) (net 2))
 (via (at 193.3 85.5) (size 0.8) (drill 0.4) (layers "F.Cu" "B.Cu") (free yes) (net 2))
 (via (at 104.8 78) (size 0.8) (drill 0.4) (layers "F.Cu" "B.Cu") (free yes) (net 2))
 (via (at 104.9 101.9) (size 0.8) (drill 0.4) (layers "F.Cu" "B.Cu") (free yes) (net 2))
 (via (at 135 61.8) (size 0.8) (drill 0.4) (layers "F.Cu" "B.Cu") (free yes) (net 2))
 (via (at 104.8 100.5) (size 0.8) (drill 0.4) (layers "F.Cu" "B.Cu") (free yes) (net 2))
 (via (at 136.5 105.2) (size 0.8) (drill 0.4) (layers "F.Cu" "B.Cu") (free yes) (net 2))
 (via (at 138 105.2) (size 0.8) (drill 0.4) (layers "F.Cu" "B.Cu") (free yes) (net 2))
 (via (at 153 105.2) (size 0.8) (drill 0.4) (layers "F.Cu" "B.Cu") (free yes) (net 2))
 (via (at 193.3 88.5) (size 0.8) (drill 0.4) (layers "F.Cu" "B.Cu") (free yes) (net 2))
 (via (at 104.8 88.5) (size 0.8) (drill 0.4) (layers "F.Cu" "B.Cu") (free yes) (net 2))
 (via (at 193.3 97.5) (size 0.8) (drill 0.4) (layers "F.Cu" "B.Cu") (free yes) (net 2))
 (via (at 193.3 76.5) (size 0.8) (drill 0.4) (layers "F.Cu" "B.Cu") (free yes) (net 2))
 (via (at 144 105.2) (size 0.8) (drill 0.4) (layers "F.Cu" "B.Cu") (free yes) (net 2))
 (via (at 180 61.8) (size 0.8) (drill 0.4) (layers "F.Cu" "B.Cu") (free yes) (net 2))
 (via (at 177 61.8) (size 0.8) (drill 0.4) (layers "F.Cu" "B.Cu") (free yes) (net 2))
 (via (at 111 105.2) (size 0.8) (drill 0.4) (layers "F.Cu" "B.Cu") (free yes) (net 2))
 (via (at 130.5 105.2) (size 0.8) (drill 0.4) (layers "F.Cu" "B.Cu") (free yes) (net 2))
 (via (at 193.3 78) (size 0.8) (drill 0.4) (layers "F.Cu" "B.Cu") (free yes) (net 2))
 (via (at 186 105.2) (size 0.8) (drill 0.4) (layers "F.Cu" "B.Cu") (free yes) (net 2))
 (via (at 104.8 91.5) (size 0.8) (drill 0.4) (layers "F.Cu" "B.Cu") (free yes) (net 2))
 (via (at 104.8 93) (size 0.8) (drill 0.4) (layers "F.Cu" "B.Cu") (free yes) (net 2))
 (via (at 112.5 105.2) (size 0.8) (drill 0.4) (layers "F.Cu" "B.Cu") (free yes) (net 2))
 (via (at 117 105.2) (size 0.8) (drill 0.4) (layers "F.Cu" "B.Cu") (free yes) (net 2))
 (via (at 108 105.1) (size 0.8) (drill 0.4) (layers "F.Cu" "B.Cu") (free yes) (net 2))
 (via (at 189.8 105.1) (size 0.8) (drill 0.4) (layers "F.Cu" "B.Cu") (free yes) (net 2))
 (via (at 156 105.2) (size 0.8) (drill 0.4) (layers "F.Cu" "B.Cu") (free yes) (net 2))
 (via (at 183 105.2) (size 0.8) (drill 0.4) (layers "F.Cu" "B.Cu") (free yes) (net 2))
 (via (at 178.5 61.8) (size 0.8) (drill 0.4) (layers "F.Cu" "B.Cu") (free yes) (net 2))
 (via (at 181.5 105.2) (size 0.8) (drill 0.4) (layers "F.Cu" "B.Cu") (free yes) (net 2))
 (via (at 104.8 94.5) (size 0.8) (drill 0.4) (layers "F.Cu" "B.Cu") (free yes) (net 2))
 (segment (start 127.25 77.75) (end 130.975 77.75) (width 1) (layer "F.Cu") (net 3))
 (segment (start 112 77.92) (end 112.17 77.75) (width 1) (layer "F.Cu") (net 3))
 (segment (start 127 86.45) (end 127 82.25) (width 1) (layer "F.Cu") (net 3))
 (segment (start 112.17 77.75) (end 127.25 77.75) (width 1) (layer "F.Cu") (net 3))
 (segment (start 123.025 77.75) (end 127.25 77.75) (width 1) (layer "F.Cu") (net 3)))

